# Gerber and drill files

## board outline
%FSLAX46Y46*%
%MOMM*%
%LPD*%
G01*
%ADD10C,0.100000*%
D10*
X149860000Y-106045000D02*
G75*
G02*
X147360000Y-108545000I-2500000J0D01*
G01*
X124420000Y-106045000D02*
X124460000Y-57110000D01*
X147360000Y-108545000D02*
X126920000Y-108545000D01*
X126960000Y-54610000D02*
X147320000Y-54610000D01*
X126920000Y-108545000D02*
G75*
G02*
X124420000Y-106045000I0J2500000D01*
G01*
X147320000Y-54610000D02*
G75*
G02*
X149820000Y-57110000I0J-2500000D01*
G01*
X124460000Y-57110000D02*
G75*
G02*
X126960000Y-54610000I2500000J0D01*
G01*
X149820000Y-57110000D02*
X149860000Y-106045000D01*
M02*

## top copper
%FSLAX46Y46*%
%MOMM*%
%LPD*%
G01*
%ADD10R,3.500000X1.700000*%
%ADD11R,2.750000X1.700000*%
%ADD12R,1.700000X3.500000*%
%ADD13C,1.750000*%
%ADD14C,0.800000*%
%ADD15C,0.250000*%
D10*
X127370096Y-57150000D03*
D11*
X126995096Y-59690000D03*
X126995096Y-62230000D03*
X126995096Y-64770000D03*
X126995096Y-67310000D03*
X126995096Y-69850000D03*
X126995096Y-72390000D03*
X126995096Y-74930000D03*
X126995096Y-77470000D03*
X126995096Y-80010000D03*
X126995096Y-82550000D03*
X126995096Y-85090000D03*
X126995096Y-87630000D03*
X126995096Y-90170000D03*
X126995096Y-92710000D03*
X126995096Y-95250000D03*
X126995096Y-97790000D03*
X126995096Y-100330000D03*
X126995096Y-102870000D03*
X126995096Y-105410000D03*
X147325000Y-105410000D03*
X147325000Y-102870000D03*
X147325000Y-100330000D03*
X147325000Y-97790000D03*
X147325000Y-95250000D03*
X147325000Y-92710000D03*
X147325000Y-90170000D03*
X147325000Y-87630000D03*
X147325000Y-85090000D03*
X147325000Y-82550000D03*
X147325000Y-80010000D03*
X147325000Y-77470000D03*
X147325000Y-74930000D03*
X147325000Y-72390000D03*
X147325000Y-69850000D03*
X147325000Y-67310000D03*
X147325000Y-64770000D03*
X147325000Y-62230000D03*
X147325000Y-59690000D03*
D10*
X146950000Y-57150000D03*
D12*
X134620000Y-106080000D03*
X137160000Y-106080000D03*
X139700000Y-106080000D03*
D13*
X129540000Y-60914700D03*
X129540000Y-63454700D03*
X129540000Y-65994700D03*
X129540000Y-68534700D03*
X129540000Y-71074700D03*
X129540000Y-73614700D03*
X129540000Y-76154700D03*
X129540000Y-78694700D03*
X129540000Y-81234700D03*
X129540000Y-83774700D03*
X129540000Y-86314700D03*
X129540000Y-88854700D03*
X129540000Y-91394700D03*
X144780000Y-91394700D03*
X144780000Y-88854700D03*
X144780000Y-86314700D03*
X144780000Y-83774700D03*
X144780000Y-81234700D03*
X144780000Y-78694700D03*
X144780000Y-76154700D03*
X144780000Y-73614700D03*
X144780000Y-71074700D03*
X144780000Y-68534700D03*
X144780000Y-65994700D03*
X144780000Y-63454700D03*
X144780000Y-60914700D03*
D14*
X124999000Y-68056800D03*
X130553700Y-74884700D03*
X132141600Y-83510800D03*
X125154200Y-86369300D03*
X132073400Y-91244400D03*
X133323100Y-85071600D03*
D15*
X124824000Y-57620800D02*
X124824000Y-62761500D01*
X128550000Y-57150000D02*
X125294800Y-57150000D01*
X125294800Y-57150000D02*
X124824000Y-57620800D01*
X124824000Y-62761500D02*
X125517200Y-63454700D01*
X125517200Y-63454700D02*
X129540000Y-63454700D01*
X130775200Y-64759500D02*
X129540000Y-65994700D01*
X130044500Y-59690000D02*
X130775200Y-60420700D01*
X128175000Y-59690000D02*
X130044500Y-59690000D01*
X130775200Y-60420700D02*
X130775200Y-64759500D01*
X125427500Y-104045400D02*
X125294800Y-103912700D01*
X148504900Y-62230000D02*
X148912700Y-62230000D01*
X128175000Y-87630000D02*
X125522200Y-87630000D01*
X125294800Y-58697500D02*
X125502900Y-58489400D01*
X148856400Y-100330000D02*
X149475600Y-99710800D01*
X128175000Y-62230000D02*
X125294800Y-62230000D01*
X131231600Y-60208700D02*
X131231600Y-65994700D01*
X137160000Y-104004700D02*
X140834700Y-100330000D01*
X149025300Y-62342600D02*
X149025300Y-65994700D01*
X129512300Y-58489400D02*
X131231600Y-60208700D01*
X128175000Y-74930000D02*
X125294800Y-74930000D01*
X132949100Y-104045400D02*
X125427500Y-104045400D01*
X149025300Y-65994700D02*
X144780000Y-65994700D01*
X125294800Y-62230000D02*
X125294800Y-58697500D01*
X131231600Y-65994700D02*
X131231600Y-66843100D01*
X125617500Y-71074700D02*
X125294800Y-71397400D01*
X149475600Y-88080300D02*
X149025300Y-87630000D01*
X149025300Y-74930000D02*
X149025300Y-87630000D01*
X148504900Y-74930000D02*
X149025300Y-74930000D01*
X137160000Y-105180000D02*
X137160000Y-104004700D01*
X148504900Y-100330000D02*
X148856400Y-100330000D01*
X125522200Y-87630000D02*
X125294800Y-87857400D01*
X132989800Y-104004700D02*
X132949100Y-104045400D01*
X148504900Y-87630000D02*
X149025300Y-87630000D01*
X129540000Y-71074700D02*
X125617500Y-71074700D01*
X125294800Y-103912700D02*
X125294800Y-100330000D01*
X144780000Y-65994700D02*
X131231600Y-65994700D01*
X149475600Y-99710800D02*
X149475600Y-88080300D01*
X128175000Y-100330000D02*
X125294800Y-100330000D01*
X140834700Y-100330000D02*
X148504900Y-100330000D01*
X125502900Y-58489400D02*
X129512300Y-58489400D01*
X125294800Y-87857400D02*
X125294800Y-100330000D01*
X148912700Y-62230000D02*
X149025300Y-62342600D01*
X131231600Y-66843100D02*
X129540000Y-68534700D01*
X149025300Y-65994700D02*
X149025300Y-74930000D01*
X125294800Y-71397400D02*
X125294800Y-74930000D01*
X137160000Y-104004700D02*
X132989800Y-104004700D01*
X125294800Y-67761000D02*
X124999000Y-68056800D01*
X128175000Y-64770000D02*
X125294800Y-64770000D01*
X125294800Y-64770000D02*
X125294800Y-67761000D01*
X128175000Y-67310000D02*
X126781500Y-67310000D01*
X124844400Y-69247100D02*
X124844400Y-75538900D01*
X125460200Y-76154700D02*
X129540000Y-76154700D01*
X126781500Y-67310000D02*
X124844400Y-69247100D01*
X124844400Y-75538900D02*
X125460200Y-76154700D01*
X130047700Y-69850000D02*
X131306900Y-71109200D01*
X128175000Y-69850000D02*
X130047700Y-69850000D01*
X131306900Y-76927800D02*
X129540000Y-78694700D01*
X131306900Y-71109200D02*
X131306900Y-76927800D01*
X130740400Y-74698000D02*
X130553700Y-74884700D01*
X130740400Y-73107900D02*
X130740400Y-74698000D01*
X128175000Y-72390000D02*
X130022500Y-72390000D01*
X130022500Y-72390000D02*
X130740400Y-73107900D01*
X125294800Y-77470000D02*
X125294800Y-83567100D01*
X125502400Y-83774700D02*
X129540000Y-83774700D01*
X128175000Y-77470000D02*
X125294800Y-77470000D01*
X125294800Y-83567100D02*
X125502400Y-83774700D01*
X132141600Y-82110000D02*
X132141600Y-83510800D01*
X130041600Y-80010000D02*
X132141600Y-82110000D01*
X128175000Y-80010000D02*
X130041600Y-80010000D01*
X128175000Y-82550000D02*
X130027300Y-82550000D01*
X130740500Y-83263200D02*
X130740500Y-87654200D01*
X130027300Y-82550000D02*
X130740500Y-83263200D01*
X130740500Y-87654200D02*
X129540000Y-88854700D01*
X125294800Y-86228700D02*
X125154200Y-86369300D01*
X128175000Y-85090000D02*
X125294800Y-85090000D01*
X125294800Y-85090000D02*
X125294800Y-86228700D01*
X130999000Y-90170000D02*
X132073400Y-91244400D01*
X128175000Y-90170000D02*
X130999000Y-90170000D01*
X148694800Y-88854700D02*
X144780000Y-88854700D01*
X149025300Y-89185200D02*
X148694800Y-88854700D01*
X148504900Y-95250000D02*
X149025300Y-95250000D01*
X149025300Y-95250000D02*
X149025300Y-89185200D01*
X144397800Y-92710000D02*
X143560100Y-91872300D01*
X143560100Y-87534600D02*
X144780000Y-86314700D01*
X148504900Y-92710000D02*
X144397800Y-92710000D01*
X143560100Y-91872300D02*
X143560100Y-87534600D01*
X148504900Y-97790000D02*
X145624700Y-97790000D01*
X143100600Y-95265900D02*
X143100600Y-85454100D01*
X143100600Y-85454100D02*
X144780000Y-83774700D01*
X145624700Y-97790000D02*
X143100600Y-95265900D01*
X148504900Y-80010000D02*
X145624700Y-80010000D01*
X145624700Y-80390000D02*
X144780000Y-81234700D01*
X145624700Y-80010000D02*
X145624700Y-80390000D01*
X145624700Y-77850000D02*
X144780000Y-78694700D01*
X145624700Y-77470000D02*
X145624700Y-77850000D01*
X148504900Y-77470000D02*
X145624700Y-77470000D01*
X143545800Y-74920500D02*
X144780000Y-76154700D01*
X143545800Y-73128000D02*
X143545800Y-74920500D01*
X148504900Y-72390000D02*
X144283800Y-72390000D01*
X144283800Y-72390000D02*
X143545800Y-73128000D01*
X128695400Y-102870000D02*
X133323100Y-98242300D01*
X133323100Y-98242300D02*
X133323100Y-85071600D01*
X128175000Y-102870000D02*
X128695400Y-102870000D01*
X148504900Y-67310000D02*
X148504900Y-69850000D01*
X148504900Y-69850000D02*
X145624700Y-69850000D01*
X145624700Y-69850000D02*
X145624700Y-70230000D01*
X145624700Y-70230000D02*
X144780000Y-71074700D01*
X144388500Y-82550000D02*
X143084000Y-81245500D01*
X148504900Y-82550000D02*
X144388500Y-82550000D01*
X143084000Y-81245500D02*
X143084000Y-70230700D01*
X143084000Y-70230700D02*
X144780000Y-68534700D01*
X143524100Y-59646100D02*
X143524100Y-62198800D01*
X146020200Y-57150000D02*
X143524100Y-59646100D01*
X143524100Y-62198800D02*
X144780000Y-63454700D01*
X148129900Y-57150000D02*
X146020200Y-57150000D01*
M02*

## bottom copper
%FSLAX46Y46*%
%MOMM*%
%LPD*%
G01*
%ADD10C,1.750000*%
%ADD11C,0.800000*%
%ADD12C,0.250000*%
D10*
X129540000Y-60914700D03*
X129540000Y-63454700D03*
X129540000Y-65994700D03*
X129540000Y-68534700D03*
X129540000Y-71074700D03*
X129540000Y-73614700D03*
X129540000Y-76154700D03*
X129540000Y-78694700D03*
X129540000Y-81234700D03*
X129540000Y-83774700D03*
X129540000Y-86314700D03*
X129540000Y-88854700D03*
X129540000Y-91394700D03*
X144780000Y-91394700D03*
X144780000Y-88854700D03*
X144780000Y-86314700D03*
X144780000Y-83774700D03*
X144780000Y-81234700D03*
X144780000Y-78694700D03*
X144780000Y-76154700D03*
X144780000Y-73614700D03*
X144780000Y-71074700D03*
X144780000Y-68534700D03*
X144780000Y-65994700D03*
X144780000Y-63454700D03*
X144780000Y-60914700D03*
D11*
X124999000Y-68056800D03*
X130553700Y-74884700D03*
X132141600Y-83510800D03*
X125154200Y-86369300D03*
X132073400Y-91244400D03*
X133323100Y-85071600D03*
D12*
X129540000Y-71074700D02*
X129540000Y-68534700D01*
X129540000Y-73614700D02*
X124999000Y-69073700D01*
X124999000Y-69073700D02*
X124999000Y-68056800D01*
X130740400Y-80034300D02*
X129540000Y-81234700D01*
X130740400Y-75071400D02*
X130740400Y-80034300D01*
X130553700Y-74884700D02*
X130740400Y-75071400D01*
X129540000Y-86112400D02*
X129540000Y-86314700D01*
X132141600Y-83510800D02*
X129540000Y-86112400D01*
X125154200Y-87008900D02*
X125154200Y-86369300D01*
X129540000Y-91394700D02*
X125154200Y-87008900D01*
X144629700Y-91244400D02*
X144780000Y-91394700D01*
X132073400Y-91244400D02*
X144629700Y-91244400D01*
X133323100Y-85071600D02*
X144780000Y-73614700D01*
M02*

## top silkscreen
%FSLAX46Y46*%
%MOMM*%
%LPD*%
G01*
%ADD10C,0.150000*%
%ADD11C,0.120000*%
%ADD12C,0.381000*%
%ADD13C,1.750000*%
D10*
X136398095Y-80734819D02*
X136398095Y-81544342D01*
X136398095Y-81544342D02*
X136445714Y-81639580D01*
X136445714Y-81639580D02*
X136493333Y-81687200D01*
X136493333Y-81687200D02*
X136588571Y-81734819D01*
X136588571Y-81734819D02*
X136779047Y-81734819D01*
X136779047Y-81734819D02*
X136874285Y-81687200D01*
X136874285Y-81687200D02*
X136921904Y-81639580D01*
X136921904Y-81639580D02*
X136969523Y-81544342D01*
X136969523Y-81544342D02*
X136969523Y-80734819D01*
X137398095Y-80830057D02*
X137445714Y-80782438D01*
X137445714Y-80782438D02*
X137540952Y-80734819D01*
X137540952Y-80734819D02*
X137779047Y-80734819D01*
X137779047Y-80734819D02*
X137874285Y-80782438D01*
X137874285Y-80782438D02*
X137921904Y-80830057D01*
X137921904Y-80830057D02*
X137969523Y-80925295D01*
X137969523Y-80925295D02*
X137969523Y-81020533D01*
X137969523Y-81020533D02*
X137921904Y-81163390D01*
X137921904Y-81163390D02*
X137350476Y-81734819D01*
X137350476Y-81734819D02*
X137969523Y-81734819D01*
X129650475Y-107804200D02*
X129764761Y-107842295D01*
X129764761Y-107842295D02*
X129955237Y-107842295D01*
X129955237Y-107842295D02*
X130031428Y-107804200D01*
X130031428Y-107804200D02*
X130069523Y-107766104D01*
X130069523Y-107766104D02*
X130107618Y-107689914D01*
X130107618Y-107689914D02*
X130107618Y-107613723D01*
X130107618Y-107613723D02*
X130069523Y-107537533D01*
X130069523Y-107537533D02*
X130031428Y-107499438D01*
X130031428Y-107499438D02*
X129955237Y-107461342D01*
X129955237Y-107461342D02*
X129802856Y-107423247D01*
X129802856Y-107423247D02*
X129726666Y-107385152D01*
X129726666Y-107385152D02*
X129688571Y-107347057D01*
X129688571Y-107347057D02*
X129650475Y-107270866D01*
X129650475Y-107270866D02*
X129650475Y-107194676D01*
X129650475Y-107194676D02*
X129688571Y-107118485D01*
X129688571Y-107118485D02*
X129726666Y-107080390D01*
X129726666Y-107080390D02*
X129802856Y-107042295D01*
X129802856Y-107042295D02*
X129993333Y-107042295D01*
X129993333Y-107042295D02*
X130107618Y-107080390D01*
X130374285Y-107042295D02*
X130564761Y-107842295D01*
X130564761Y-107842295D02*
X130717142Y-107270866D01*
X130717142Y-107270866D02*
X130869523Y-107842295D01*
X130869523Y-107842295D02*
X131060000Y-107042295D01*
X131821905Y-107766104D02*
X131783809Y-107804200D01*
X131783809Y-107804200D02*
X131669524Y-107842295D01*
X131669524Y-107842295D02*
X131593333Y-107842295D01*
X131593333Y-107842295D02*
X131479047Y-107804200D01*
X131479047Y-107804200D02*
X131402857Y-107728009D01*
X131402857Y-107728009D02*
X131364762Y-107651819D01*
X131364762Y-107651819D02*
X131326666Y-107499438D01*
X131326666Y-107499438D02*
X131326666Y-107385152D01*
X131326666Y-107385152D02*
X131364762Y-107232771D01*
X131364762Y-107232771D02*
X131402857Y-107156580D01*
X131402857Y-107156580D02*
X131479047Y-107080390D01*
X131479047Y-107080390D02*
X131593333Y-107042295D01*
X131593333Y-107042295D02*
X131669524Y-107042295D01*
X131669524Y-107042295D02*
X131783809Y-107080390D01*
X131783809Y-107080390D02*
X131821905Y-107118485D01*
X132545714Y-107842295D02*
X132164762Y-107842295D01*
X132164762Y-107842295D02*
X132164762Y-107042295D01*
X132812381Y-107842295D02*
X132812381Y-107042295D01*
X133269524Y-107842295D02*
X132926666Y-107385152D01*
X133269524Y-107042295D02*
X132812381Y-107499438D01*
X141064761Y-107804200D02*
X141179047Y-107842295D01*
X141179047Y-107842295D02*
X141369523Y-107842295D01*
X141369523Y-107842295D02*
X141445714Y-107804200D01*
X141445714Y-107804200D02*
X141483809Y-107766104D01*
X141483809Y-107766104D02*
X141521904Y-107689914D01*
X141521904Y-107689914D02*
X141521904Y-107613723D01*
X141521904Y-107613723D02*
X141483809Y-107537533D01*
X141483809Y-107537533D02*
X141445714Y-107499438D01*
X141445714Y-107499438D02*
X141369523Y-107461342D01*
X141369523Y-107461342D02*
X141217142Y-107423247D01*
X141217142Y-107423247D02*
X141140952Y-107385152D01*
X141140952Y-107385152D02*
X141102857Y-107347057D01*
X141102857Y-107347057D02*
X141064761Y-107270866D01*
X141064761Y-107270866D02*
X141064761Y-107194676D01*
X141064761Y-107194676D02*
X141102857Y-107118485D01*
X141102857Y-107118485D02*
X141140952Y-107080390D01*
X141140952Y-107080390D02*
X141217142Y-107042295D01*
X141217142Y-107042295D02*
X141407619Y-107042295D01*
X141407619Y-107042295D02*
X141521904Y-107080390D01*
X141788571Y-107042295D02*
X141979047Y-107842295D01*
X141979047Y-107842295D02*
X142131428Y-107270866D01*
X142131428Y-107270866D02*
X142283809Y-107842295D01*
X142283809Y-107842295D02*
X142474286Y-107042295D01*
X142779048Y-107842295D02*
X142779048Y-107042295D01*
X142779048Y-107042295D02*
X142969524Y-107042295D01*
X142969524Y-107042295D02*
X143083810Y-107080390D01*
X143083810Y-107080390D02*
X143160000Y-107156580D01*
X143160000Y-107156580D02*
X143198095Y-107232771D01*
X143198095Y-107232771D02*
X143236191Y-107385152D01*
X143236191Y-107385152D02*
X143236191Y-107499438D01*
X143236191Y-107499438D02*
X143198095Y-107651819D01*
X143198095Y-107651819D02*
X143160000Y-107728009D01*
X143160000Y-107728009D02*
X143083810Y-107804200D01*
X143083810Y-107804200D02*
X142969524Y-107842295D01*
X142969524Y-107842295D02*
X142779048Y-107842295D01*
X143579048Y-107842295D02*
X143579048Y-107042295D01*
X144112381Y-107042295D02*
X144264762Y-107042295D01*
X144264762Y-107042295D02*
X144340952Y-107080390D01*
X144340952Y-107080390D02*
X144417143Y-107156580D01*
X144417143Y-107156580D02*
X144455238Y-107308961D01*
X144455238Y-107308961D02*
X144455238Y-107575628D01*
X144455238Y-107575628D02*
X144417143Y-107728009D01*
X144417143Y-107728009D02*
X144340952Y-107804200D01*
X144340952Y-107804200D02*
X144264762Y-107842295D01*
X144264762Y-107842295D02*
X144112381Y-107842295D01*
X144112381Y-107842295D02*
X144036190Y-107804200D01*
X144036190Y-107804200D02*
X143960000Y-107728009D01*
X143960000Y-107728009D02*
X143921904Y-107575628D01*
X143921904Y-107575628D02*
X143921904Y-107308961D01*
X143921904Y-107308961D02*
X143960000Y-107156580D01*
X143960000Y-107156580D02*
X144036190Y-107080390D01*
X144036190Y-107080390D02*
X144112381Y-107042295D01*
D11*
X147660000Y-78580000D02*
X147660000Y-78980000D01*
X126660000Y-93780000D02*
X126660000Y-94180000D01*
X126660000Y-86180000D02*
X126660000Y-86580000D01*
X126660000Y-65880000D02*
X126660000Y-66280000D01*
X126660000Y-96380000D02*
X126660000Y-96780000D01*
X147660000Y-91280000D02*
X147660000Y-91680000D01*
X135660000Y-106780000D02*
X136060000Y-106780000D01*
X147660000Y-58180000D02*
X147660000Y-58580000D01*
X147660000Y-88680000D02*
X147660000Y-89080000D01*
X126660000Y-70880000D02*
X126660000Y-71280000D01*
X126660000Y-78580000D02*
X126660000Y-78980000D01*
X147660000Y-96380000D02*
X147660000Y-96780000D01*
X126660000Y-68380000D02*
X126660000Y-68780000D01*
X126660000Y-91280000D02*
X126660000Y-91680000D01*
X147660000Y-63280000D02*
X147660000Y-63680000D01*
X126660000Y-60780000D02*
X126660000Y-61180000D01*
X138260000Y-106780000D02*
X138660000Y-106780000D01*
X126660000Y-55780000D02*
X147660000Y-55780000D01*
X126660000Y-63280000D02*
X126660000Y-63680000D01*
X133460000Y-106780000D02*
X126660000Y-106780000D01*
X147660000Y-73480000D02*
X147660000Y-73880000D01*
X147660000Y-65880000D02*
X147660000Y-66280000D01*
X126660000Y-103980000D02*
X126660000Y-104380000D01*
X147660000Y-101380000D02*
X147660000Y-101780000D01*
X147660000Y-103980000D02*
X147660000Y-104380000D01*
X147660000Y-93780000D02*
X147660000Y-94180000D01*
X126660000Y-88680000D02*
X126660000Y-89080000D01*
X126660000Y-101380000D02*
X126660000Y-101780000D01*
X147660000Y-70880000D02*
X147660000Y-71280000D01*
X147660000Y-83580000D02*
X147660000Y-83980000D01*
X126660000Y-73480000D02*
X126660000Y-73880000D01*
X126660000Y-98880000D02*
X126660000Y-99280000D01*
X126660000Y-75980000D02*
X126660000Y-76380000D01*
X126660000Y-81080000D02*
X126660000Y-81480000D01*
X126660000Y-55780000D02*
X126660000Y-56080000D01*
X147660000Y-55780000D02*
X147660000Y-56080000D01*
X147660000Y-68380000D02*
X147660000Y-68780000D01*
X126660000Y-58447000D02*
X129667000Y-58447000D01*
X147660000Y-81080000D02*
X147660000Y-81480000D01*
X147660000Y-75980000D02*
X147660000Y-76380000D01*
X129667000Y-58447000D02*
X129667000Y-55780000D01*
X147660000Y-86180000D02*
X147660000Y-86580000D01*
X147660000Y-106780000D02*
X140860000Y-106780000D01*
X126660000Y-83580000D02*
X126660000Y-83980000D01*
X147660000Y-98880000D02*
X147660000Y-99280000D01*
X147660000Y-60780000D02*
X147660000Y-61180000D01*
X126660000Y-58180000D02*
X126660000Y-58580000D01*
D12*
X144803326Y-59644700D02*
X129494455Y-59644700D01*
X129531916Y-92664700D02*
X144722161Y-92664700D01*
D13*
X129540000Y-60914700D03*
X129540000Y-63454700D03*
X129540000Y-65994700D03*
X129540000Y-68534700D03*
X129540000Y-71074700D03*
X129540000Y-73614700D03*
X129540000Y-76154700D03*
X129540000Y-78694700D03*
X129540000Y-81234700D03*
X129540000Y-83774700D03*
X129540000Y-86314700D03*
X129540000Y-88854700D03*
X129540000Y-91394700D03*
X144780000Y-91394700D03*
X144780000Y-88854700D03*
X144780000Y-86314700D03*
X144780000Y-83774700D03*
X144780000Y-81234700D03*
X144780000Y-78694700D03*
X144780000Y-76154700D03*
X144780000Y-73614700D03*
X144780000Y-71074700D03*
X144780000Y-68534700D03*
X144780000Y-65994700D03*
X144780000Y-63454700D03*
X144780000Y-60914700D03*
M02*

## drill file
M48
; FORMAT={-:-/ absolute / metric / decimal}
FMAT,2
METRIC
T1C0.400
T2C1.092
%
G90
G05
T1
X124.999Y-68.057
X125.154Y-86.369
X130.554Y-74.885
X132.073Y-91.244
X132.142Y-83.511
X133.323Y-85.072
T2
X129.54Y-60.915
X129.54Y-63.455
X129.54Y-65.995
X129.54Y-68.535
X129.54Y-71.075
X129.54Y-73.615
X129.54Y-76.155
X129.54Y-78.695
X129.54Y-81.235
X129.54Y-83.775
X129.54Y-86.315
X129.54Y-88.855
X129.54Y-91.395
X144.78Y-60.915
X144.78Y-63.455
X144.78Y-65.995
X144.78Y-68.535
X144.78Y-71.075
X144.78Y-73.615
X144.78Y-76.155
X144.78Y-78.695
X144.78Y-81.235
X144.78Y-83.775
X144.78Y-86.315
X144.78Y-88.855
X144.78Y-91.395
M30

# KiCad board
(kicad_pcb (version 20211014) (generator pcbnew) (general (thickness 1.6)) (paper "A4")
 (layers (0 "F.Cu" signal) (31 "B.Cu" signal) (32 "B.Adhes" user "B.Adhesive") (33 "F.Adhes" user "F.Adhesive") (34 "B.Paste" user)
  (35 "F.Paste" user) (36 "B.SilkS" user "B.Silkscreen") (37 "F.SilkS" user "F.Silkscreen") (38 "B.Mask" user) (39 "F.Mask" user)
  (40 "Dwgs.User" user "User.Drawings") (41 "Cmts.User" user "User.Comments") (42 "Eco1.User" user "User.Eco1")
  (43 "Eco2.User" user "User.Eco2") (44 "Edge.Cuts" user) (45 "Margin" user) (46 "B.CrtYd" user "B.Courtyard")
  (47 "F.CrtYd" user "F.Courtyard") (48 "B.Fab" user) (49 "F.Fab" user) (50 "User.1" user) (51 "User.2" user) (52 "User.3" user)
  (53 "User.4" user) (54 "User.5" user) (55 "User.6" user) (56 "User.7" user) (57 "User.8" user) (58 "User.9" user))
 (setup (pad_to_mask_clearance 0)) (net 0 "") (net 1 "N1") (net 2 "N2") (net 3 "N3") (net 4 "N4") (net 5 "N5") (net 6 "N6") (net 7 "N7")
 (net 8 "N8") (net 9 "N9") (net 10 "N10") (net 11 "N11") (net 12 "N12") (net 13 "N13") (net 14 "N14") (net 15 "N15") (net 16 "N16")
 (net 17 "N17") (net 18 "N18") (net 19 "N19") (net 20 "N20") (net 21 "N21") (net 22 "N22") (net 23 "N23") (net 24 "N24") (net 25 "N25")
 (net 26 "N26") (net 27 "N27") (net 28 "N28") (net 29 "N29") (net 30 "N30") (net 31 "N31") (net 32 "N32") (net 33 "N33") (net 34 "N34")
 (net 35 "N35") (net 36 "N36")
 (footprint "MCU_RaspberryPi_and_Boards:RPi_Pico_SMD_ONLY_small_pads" (layer "F.Cu") (at 137.16 81.28)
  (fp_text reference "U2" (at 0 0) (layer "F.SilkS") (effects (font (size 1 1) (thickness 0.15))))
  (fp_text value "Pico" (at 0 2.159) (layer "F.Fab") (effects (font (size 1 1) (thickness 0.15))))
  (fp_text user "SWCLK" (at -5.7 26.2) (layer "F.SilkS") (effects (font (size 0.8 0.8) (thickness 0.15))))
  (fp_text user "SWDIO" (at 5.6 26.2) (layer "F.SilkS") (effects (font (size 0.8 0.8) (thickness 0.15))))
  (fp_line (start 10.5 -2.7) (end 10.5 -2.3) (layer "F.SilkS") (width 0.12))
  (fp_line (start -10.5 12.5) (end -10.5 12.9) (layer "F.SilkS") (width 0.12))
  (fp_line (start -10.5 4.9) (end -10.5 5.3) (layer "F.SilkS") (width 0.12))
  (fp_line (start -10.5 -15.4) (end -10.5 -15) (layer "F.SilkS") (width 0.12))
  (fp_line (start -10.5 15.1) (end -10.5 15.5) (layer "F.SilkS") (width 0.12))
  (fp_line (start 10.5 10) (end 10.5 10.4) (layer "F.SilkS") (width 0.12))
  (fp_line (start -1.5 25.5) (end -1.1 25.5) (layer "F.SilkS") (width 0.12))
  (fp_line (start 10.5 -23.1) (end 10.5 -22.7) (layer "F.SilkS") (width 0.12))
  (fp_line (start 10.5 7.4) (end 10.5 7.8) (layer "F.SilkS") (width 0.12))
  (fp_line (start -10.5 -10.4) (end -10.5 -10) (layer "F.SilkS") (width 0.12))
  (fp_line (start -10.5 -2.7) (end -10.5 -2.3) (layer "F.SilkS") (width 0.12))
  (fp_line (start 10.5 15.1) (end 10.5 15.5) (layer "F.SilkS") (width 0.12))
  (fp_line (start -10.5 -12.9) (end -10.5 -12.5) (layer "F.SilkS") (width 0.12))
  (fp_line (start -10.5 10) (end -10.5 10.4) (layer "F.SilkS") (width 0.12))
  (fp_line (start 10.5 -18) (end 10.5 -17.6) (layer "F.SilkS") (width 0.12))
  (fp_line (start -10.5 -20.5) (end -10.5 -20.1) (layer "F.SilkS") (width 0.12))
  (fp_line (start 1.1 25.5) (end 1.5 25.5) (layer "F.SilkS") (width 0.12))
  (fp_line (start -10.5 -25.5) (end 10.5 -25.5) (layer "F.SilkS") (width 0.12))
  (fp_line (start -10.5 -18) (end -10.5 -17.6) (layer "F.SilkS") (width 0.12))
  (fp_line (start -3.7 25.5) (end -10.5 25.5) (layer "F.SilkS") (width 0.12))
  (fp_line (start 10.5 -7.8) (end 10.5 -7.4) (layer "F.SilkS") (width 0.12))
  (fp_line (start 10.5 -15.4) (end 10.5 -15) (layer "F.SilkS") (width 0.12))
  (fp_line (start -10.5 22.7) (end -10.5 23.1) (layer "F.SilkS") (width 0.12))
  (fp_line (start 10.5 20.1) (end 10.5 20.5) (layer "F.SilkS") (width 0.12))
  (fp_line (start 10.5 22.7) (end 10.5 23.1) (layer "F.SilkS") (width 0.12))
  (fp_line (start 10.5 12.5) (end 10.5 12.9) (layer "F.SilkS") (width 0.12))
  (fp_line (start -10.5 7.4) (end -10.5 7.8) (layer "F.SilkS") (width 0.12))
  (fp_line (start -10.5 20.1) (end -10.5 20.5) (layer "F.SilkS") (width 0.12))
  (fp_line (start 10.5 -10.4) (end 10.5 -10) (layer "F.SilkS") (width 0.12))
  (fp_line (start 10.5 2.3) (end 10.5 2.7) (layer "F.SilkS") (width 0.12))
  (fp_line (start -10.5 -7.8) (end -10.5 -7.4) (layer "F.SilkS") (width 0.12))
  (fp_line (start -10.5 17.6) (end -10.5 18) (layer "F.SilkS") (width 0.12))
  (fp_line (start -10.5 -5.3) (end -10.5 -4.9) (layer "F.SilkS") (width 0.12))
  (fp_line (start -10.5 -0.2) (end -10.5 0.2) (layer "F.SilkS") (width 0.12))
  (fp_line (start -10.5 -25.5) (end -10.5 -25.2) (layer "F.SilkS") (width 0.12))
  (fp_line (start 10.5 -25.5) (end 10.5 -25.2) (layer "F.SilkS") (width 0.12))
  (fp_line (start 10.5 -12.9) (end 10.5 -12.5) (layer "F.SilkS") (width 0.12))
  (fp_line (start -10.5 -22.833) (end -7.493 -22.833) (layer "F.SilkS") (width 0.12))
  (fp_line (start 10.5 -0.2) (end 10.5 0.2) (layer "F.SilkS") (width 0.12))
  (fp_line (start 10.5 -5.3) (end 10.5 -4.9) (layer "F.SilkS") (width 0.12))
  (fp_line (start -7.493 -22.833) (end -7.493 -25.5) (layer "F.SilkS") (width 0.12))
  (fp_line (start 10.5 4.9) (end 10.5 5.3) (layer "F.SilkS") (width 0.12))
  (fp_line (start 10.5 25.5) (end 3.7 25.5) (layer "F.SilkS") (width 0.12))
  (fp_line (start -10.5 2.3) (end -10.5 2.7) (layer "F.SilkS") (width 0.12))
  (fp_line (start 10.5 17.6) (end 10.5 18) (layer "F.SilkS") (width 0.12))
  (fp_line (start 10.5 -20.5) (end 10.5 -20.1) (layer "F.SilkS") (width 0.12))
  (fp_line (start -10.5 -23.1) (end -10.5 -22.7) (layer "F.SilkS") (width 0.12))
  (pad "1" smd rect (at -8.609992 -24.13) (size 3.5 1.7) (drill (offset -1.179912 0)) (layers "F.Cu" "F.Mask") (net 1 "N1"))
  (pad "2" smd rect (at -8.984992 -21.59) (size 2.75 1.7) (drill (offset -1.179912 0)) (layers "F.Cu" "F.Mask") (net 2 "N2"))
  (pad "3" smd rect (at -8.984992 -19.05) (size 2.75 1.7) (drill (offset -1.179912 0)) (layers "F.Cu" "F.Mask") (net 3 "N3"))
  (pad "4" smd rect (at -8.984992 -16.51) (size 2.75 1.7) (drill (offset -1.179912 0)) (layers "F.Cu" "F.Mask") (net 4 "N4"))
  (pad "5" smd rect (at -8.984992 -13.97) (size 2.75 1.7) (drill (offset -1.179912 0)) (layers "F.Cu" "F.Mask") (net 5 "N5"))
  (pad "6" smd rect (at -8.984992 -11.43) (size 2.75 1.7) (drill (offset -1.179912 0)) (layers "F.Cu" "F.Mask") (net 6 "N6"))
  (pad "7" smd rect (at -8.984992 -8.89) (size 2.75 1.7) (drill (offset -1.179912 0)) (layers "F.Cu" "F.Mask") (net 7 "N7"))
  (pad "8" smd rect (at -8.984992 -6.35) (size 2.75 1.7) (drill (offset -1.179912 0)) (layers "F.Cu" "F.Mask") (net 3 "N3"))
  (pad "9" smd rect (at -8.984992 -3.81) (size 2.75 1.7) (drill (offset -1.179912 0)) (layers "F.Cu" "F.Mask") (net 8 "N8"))
  (pad "10" smd rect (at -8.984992 -1.27) (size 2.75 1.7) (drill (offset -1.179912 0)) (layers "F.Cu" "F.Mask") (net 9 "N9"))
  (pad "11" smd rect (at -8.984992 1.27) (size 2.75 1.7) (drill (offset -1.179912 0)) (layers "F.Cu" "F.Mask") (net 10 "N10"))
  (pad "12" smd rect (at -8.984992 3.81) (size 2.75 1.7) (drill (offset -1.179912 0)) (layers "F.Cu" "F.Mask") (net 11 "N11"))
  (pad "13" smd rect (at -8.984992 6.35) (size 2.75 1.7) (drill (offset -1.179912 0)) (layers "F.Cu" "F.Mask") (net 3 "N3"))
  (pad "14" smd rect (at -8.984992 8.89) (size 2.75 1.7) (drill (offset -1.179912 0)) (layers "F.Cu" "F.Mask") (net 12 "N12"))
  (pad "15" smd rect (at -8.984992 11.43) (size 2.75 1.7) (drill (offset -1.179912 0)) (layers "F.Cu" "F.Mask") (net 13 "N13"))
  (pad "16" smd rect (at -8.984992 13.97) (size 2.75 1.7) (drill (offset -1.179912 0)) (layers "F.Cu" "F.Mask") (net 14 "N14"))
  (pad "17" smd rect (at -8.984992 16.51) (size 2.75 1.7) (drill (offset -1.179912 0)) (layers "F.Cu" "F.Mask") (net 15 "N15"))
  (pad "18" smd rect (at -8.984992 19.05) (size 2.75 1.7) (drill (offset -1.179912 0)) (layers "F.Cu" "F.Mask") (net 3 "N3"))
  (pad "19" smd rect (at -8.984992 21.59) (size 2.75 1.7) (drill (offset -1.179912 0)) (layers "F.Cu" "F.Mask") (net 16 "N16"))
  (pad "20" smd rect (at -8.984992 24.13) (size 2.75 1.7) (drill (offset -1.179912 0)) (layers "F.Cu" "F.Mask") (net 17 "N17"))
  (pad "21" smd rect (at 11.344912 24.13) (size 2.75 1.7) (drill (offset -1.179912 0)) (layers "F.Cu" "F.Mask") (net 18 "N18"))
  (pad "22" smd rect (at 11.344912 21.59) (size 2.75 1.7) (drill (offset -1.179912 0)) (layers "F.Cu" "F.Mask") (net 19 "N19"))
  (pad "23" smd rect (at 11.344912 19.05) (size 2.75 1.7) (drill (offset -1.179912 0)) (layers "F.Cu" "F.Mask") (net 3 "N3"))
  (pad "24" smd rect (at 11.344912 16.51) (size 2.75 1.7) (drill (offset -1.179912 0)) (layers "F.Cu" "F.Mask") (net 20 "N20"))
  (pad "25" smd rect (at 11.344912 13.97) (size 2.75 1.7) (drill (offset -1.179912 0)) (layers "F.Cu" "F.Mask") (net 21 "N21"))
  (pad "26" smd rect (at 11.344912 11.43) (size 2.75 1.7) (drill (offset -1.179912 0)) (layers "F.Cu" "F.Mask") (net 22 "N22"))
  (pad "27" smd rect (at 11.344912 8.89) (size 2.75 1.7) (drill (offset -1.179912 0)) (layers "F.Cu" "F.Mask") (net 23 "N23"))
  (pad "28" smd rect (at 11.344912 6.35) (size 2.75 1.7) (drill (offset -1.179912 0)) (layers "F.Cu" "F.Mask") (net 3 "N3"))
  (pad "29" smd rect (at 11.344912 3.81) (size 2.75 1.7) (drill (offset -1.179912 0)) (layers "F.Cu" "F.Mask") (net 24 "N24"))
  (pad "30" smd rect (at 11.344912 1.27) (size 2.75 1.7) (drill (offset -1.179912 0)) (layers "F.Cu" "F.Mask") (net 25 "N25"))
  (pad "31" smd rect (at 11.344912 -1.27) (size 2.75 1.7) (drill (offset -1.179912 0)) (layers "F.Cu" "F.Mask") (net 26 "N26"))
  (pad "32" smd rect (at 11.344912 -3.81) (size 2.75 1.7) (drill (offset -1.179912 0)) (layers "F.Cu" "F.Mask") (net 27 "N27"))
  (pad "33" smd rect (at 11.344912 -6.35) (size 2.75 1.7) (drill (offset -1.179912 0)) (layers "F.Cu" "F.Mask") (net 3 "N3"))
  (pad "34" smd rect (at 11.344912 -8.89) (size 2.75 1.7) (drill (offset -1.179912 0)) (layers "F.Cu" "F.Mask") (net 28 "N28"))
  (pad "35" smd rect (at 11.344912 -11.43) (size 2.75 1.7) (drill (offset -1.179912 0)) (layers "F.Cu" "F.Mask") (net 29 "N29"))
  (pad "36" smd rect (at 11.344912 -13.97) (size 2.75 1.7) (drill (offset -1.179912 0)) (layers "F.Cu" "F.Mask") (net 29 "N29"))
  (pad "37" smd rect (at 11.344912 -16.51) (size 2.75 1.7) (drill (offset -1.179912 0)) (layers "F.Cu" "F.Mask") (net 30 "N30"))
  (pad "38" smd rect (at 11.344912 -19.05) (size 2.75 1.7) (drill (offset -1.179912 0)) (layers "F.Cu" "F.Mask") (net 3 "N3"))
  (pad "39" smd rect (at 11.344912 -21.59) (size 2.75 1.7) (drill (offset -1.179912 0)) (layers "F.Cu" "F.Mask") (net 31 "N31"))
  (pad "40" smd rect (at 10.969912 -24.13) (size 3.5 1.7) (drill (offset -1.179912 0)) (layers "F.Cu" "F.Mask") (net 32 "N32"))
  (pad "41" smd rect (at -2.54 23.9 90) (size 3.5 1.7) (drill (offset -0.9 0)) (layers "F.Cu" "F.Mask") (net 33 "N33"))
  (pad "42" smd rect (at 0 23.9 90) (size 3.5 1.7) (drill (offset -0.9 0)) (layers "F.Cu" "F.Mask") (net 3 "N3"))
  (pad "43" smd rect (at 2.54 23.9 90) (size 3.5 1.7) (drill (offset -0.9 0)) (layers "F.Cu" "F.Mask") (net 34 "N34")))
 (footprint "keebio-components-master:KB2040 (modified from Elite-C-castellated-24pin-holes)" (layer "B.Cu") (at 137.16 77.4247 -90)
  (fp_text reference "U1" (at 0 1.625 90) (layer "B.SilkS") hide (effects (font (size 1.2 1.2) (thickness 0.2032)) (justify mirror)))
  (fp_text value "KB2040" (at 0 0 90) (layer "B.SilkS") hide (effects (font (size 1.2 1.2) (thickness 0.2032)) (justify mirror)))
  (fp_line (start -17.78 -7.643326) (end -17.78 7.665545) (layer "F.SilkS") (width 0.381))
  (fp_line (start 15.24 7.628084) (end 15.24 -7.562161) (layer "F.SilkS") (width 0.381))
  (pad "0" thru_hole circle (at -16.51 7.62 90) (size 1.75 1.75) (drill 1.0922) (layers *.Cu *.SilkS *.Mask) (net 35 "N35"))
  (pad "1" thru_hole circle (at -13.97 7.62 90) (size 1.75 1.75) (drill 1.0922) (layers *.Cu *.SilkS *.Mask) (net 1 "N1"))
  (pad "2" thru_hole circle (at -11.43 7.62 90) (size 1.75 1.75) (drill 1.0922) (layers *.Cu *.SilkS *.Mask) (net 2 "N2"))
  (pad "3" thru_hole circle (at -8.89 7.62 90) (size 1.75 1.75) (drill 1.0922) (layers *.Cu *.SilkS *.Mask) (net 3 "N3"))
  (pad "4" thru_hole circle (at -6.35 7.62 90) (size 1.75 1.75) (drill 1.0922) (layers *.Cu *.SilkS *.Mask) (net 3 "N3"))
  (pad "5" thru_hole circle (at -3.81 7.62 90) (size 1.75 1.75) (drill 1.0922) (layers *.Cu *.SilkS *.Mask) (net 4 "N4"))
  (pad "6" thru_hole circle (at -1.27 7.62 90) (size 1.75 1.75) (drill 1.0922) (layers *.Cu *.SilkS *.Mask) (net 5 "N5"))
  (pad "7" thru_hole circle (at 1.27 7.62 90) (size 1.75 1.75) (drill 1.0922) (layers *.Cu *.SilkS *.Mask) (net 6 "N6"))
  (pad "8" thru_hole circle (at 3.81 7.62 90) (size 1.75 1.75) (drill 1.0922) (layers *.Cu *.SilkS *.Mask) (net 7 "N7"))
  (pad "9" thru_hole circle (at 6.35 7.62 90) (size 1.75 1.75) (drill 1.0922) (layers *.Cu *.SilkS *.Mask) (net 8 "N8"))
  (pad "10" thru_hole circle (at 8.89 7.62 90) (size 1.75 1.75) (drill 1.0922) (layers *.Cu *.SilkS *.Mask) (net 9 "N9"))
  (pad "11" thru_hole circle (at 11.43 7.62 90) (size 1.75 1.75) (drill 1.0922) (layers *.Cu *.SilkS *.Mask) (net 10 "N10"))
  (pad "12" thru_hole circle (at 13.97 7.62 90) (size 1.75 1.75) (drill 1.0922) (layers *.Cu *.SilkS *.Mask) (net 11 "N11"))
  (pad "13" thru_hole circle (at 13.97 -7.62 90) (size 1.75 1.75) (drill 1.0922) (layers *.Cu *.SilkS *.Mask) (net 12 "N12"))
  (pad "14" thru_hole circle (at 11.43 -7.62 90) (size 1.75 1.75) (drill 1.0922) (layers *.Cu *.SilkS *.Mask) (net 21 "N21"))
  (pad "15" thru_hole circle (at 8.89 -7.62 90) (size 1.75 1.75) (drill 1.0922) (layers *.Cu *.SilkS *.Mask) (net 22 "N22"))
  (pad "16" thru_hole circle (at 6.35 -7.62 90) (size 1.75 1.75) (drill 1.0922) (layers *.Cu *.SilkS *.Mask) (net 20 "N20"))
  (pad "17" thru_hole circle (at 3.81 -7.62 90) (size 1.75 1.75) (drill 1.0922) (layers *.Cu *.SilkS *.Mask) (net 26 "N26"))
  (pad "18" thru_hole circle (at 1.27 -7.62 90) (size 1.75 1.75) (drill 1.0922) (layers *.Cu *.SilkS *.Mask) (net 27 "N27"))
  (pad "19" thru_hole circle (at -1.27 -7.62 90) (size 1.75 1.75) (drill 1.0922) (layers *.Cu *.SilkS *.Mask) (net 28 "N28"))
  (pad "20" thru_hole circle (at -3.81 -7.62 90) (size 1.75 1.75) (drill 1.0922) (layers *.Cu *.SilkS *.Mask) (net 16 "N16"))
  (pad "21" thru_hole circle (at -6.35 -7.62 90) (size 1.75 1.75) (drill 1.0922) (layers *.Cu *.SilkS *.Mask) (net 29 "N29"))
  (pad "22" thru_hole circle (at -8.89 -7.62 90) (size 1.75 1.75) (drill 1.0922) (layers *.Cu *.SilkS *.Mask) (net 25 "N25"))
  (pad "23" thru_hole circle (at -11.43 -7.62 90) (size 1.75 1.75) (drill 1.0922) (layers *.Cu *.SilkS *.Mask) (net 3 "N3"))
  (pad "24" thru_hole circle (at -13.97 -7.62 90) (size 1.75 1.75) (drill 1.0922) (layers *.Cu *.SilkS *.Mask) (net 32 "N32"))
  (pad "25" thru_hole circle (at -16.51 -7.62 90) (size 1.75 1.75) (drill 1.0922) (layers *.Cu *.SilkS *.Mask) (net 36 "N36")))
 (gr_arc (start 149.86 106.045) (mid 149.127767 107.812767) (end 147.36 108.545) (layer "Edge.Cuts") (width 0.1))
 (gr_line (start 124.42 106.045) (end 124.46 57.11) (layer "Edge.Cuts") (width 0.1))
 (gr_line (start 147.36 108.545) (end 126.92 108.545) (layer "Edge.Cuts") (width 0.1))
 (gr_line (start 126.96 54.61) (end 147.32 54.61) (layer "Edge.Cuts") (width 0.1))
 (gr_arc (start 126.92 108.545) (mid 125.152233 107.812767) (end 124.42 106.045) (layer "Edge.Cuts") (width 0.1))
 (gr_arc (start 147.32 54.61) (mid 149.087767 55.342233) (end 149.82 57.11) (layer "Edge.Cuts") (width 0.1))
 (gr_arc (start 124.46 57.11) (mid 125.192233 55.342233) (end 126.96 54.61) (layer "Edge.Cuts") (width 0.1))
 (gr_line (start 149.82 57.11) (end 149.86 106.045) (layer "Edge.Cuts") (width 0.1))
 (segment (start 124.824 57.6208) (end 124.824 62.7615) (width 0.25) (layer "F.Cu") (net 1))
 (segment (start 128.55 57.15) (end 125.2948 57.15) (width 0.25) (layer "F.Cu") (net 1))
 (segment (start 125.2948 57.15) (end 124.824 57.6208) (width 0.25) (layer "F.Cu") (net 1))
 (segment (start 124.824 62.7615) (end 125.5172 63.4547) (width 0.25) (layer "F.Cu") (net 1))
 (segment (start 125.5172 63.4547) (end 129.54 63.4547) (width 0.25) (layer "F.Cu") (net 1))
 (segment (start 130.7752 64.7595) (end 129.54 65.9947) (width 0.25) (layer "F.Cu") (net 2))
 (segment (start 130.0445 59.69) (end 130.7752 60.4207) (width 0.25) (layer "F.Cu") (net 2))
 (segment (start 128.175 59.69) (end 130.0445 59.69) (width 0.25) (layer "F.Cu") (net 2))
 (segment (start 130.7752 60.4207) (end 130.7752 64.7595) (width 0.25) (layer "F.Cu") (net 2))
 (segment (start 125.4275 104.0454) (end 125.2948 103.9127) (width 0.25) (layer "F.Cu") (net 3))
 (segment (start 148.5049 62.23) (end 148.9127 62.23) (width 0.25) (layer "F.Cu") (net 3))
 (segment (start 128.175 87.63) (end 125.5222 87.63) (width 0.25) (layer "F.Cu") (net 3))
 (segment (start 125.2948 58.6975) (end 125.5029 58.4894) (width 0.25) (layer "F.Cu") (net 3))
 (segment (start 148.8564 100.33) (end 149.4756 99.7108) (width 0.25) (layer "F.Cu") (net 3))
 (segment (start 128.175 62.23) (end 125.2948 62.23) (width 0.25) (layer "F.Cu") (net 3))
 (segment (start 131.2316 60.2087) (end 131.2316 65.9947) (width 0.25) (layer "F.Cu") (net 3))
 (segment (start 137.16 104.0047) (end 140.8347 100.33) (width 0.25) (layer "F.Cu") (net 3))
 (segment (start 149.0253 62.3426) (end 149.0253 65.9947) (width 0.25) (layer "F.Cu") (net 3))
 (segment (start 129.5123 58.4894) (end 131.2316 60.2087) (width 0.25) (layer "F.Cu") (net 3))
 (segment (start 128.175 74.93) (end 125.2948 74.93) (width 0.25) (layer "F.Cu") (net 3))
 (segment (start 132.9491 104.0454) (end 125.4275 104.0454) (width 0.25) (layer "F.Cu") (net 3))
 (segment (start 149.0253 65.9947) (end 144.78 65.9947) (width 0.25) (layer "F.Cu") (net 3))
 (segment (start 125.2948 62.23) (end 125.2948 58.6975) (width 0.25) (layer "F.Cu") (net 3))
 (segment (start 131.2316 65.9947) (end 131.2316 66.8431) (width 0.25) (layer "F.Cu") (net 3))
 (segment (start 125.6175 71.0747) (end 125.2948 71.3974) (width 0.25) (layer "F.Cu") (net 3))
 (segment (start 149.4756 88.0803) (end 149.0253 87.63) (width 0.25) (layer "F.Cu") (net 3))
 (segment (start 149.0253 74.93) (end 149.0253 87.63) (width 0.25) (layer "F.Cu") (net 3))
 (segment (start 148.5049 74.93) (end 149.0253 74.93) (width 0.25) (layer "F.Cu") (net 3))
 (segment (start 137.16 105.18) (end 137.16 104.0047) (width 0.25) (layer "F.Cu") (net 3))
 (segment (start 148.5049 100.33) (end 148.8564 100.33) (width 0.25) (layer "F.Cu") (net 3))
 (segment (start 125.5222 87.63) (end 125.2948 87.8574) (width 0.25) (layer "F.Cu") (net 3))
 (segment (start 132.9898 104.0047) (end 132.9491 104.0454) (width 0.25) (layer "F.Cu") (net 3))
 (segment (start 148.5049 87.63) (end 149.0253 87.63) (width 0.25) (layer "F.Cu") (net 3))
 (segment (start 129.54 71.0747) (end 125.6175 71.0747) (width 0.25) (layer "F.Cu") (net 3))
 (segment (start 125.2948 103.9127) (end 125.2948 100.33) (width 0.25) (layer "F.Cu") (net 3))
 (segment (start 144.78 65.9947) (end 131.2316 65.9947) (width 0.25) (layer "F.Cu") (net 3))
 (segment (start 149.4756 99.7108) (end 149.4756 88.0803) (width 0.25) (layer "F.Cu") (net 3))
 (segment (start 128.175 100.33) (end 125.2948 100.33) (width 0.25) (layer "F.Cu") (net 3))
 (segment (start 140.8347 100.33) (end 148.5049 100.33) (width 0.25) (layer "F.Cu") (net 3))
 (segment (start 125.5029 58.4894) (end 129.5123 58.4894) (width 0.25) (layer "F.Cu") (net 3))
 (segment (start 125.2948 87.8574) (end 125.2948 100.33) (width 0.25) (layer "F.Cu") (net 3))
 (segment (start 148.9127 62.23) (end 149.0253 62.3426) (width 0.25) (layer "F.Cu") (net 3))
 (segment (start 131.2316 66.8431) (end 129.54 68.5347) (width 0.25) (layer "F.Cu") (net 3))
 (segment (start 149.0253 65.9947) (end 149.0253 74.93) (width 0.25) (layer "F.Cu") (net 3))
 (segment (start 125.2948 71.3974) (end 125.2948 74.93) (width 0.25) (layer "F.Cu") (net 3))
 (segment (start 137.16 104.0047) (end 132.9898 104.0047) (width 0.25) (layer "F.Cu") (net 3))
 (segment (start 129.54 71.0747) (end 129.54 68.5347) (width 0.25) (layer "B.Cu") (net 3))
 (segment (start 125.2948 67.761) (end 124.999 68.0568) (width 0.25) (layer "F.Cu") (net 4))
 (segment (start 128.175 64.77) (end 125.2948 64.77) (width 0.25) (layer "F.Cu") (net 4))
 (segment (start 125.2948 64.77) (end 125.2948 67.761) (width 0.25) (layer "F.Cu") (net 4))
 (via (at 124.999 68.0568) (size 0.8) (drill 0.4) (layers "F.Cu" "B.Cu") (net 4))
 (segment (start 129.54 73.6147) (end 124.999 69.0737) (width 0.25) (layer "B.Cu") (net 4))
 (segment (start 124.999 69.0737) (end 124.999 68.0568) (width 0.25) (layer "B.Cu") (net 4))
 (segment (start 128.175 67.31) (end 126.7815 67.31) (width 0.25) (layer "F.Cu") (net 5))
 (segment (start 124.8444 69.2471) (end 124.8444 75.5389) (width 0.25) (layer "F.Cu") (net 5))
 (segment (start 125.4602 76.1547) (end 129.54 76.1547) (width 0.25) (layer "F.Cu") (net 5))
 (segment (start 126.7815 67.31) (end 124.8444 69.2471) (width 0.25) (layer "F.Cu") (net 5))
 (segment (start 124.8444 75.5389) (end 125.4602 76.1547) (width 0.25) (layer "F.Cu") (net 5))
 (segment (start 130.0477 69.85) (end 131.3069 71.1092) (width 0.25) (layer "F.Cu") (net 6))
 (segment (start 128.175 69.85) (end 130.0477 69.85) (width 0.25) (layer "F.Cu") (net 6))
 (segment (start 131.3069 76.9278) (end 129.54 78.6947) (width 0.25) (layer "F.Cu") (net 6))
 (segment (start 131.3069 71.1092) (end 131.3069 76.9278) (width 0.25) (layer "F.Cu") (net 6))
 (segment (start 130.7404 74.698) (end 130.5537 74.8847) (width 0.25) (layer "F.Cu") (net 7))
 (segment (start 130.7404 73.1079) (end 130.7404 74.698) (width 0.25) (layer "F.Cu") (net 7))
 (segment (start 128.175 72.39) (end 130.0225 72.39) (width 0.25) (layer "F.Cu") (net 7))
 (segment (start 130.0225 72.39) (end 130.7404 73.1079) (width 0.25) (layer "F.Cu") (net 7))
 (via (at 130.5537 74.8847) (size 0.8) (drill 0.4) (layers "F.Cu" "B.Cu") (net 7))
 (segment (start 130.7404 80.0343) (end 129.54 81.2347) (width 0.25) (layer "B.Cu") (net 7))
 (segment (start 130.7404 75.0714) (end 130.7404 80.0343) (width 0.25) (layer "B.Cu") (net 7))
 (segment (start 130.5537 74.8847) (end 130.7404 75.0714) (width 0.25) (layer "B.Cu") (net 7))
 (segment (start 125.2948 77.47) (end 125.2948 83.5671) (width 0.25) (layer "F.Cu") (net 8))
 (segment (start 125.5024 83.7747) (end 129.54 83.7747) (width 0.25) (layer "F.Cu") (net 8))
 (segment (start 128.175 77.47) (end 125.2948 77.47) (width 0.25) (layer "F.Cu") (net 8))
 (segment (start 125.2948 83.5671) (end 125.5024 83.7747) (width 0.25) (layer "F.Cu") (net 8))
 (segment (start 132.1416 82.11) (end 132.1416 83.5108) (width 0.25) (layer "F.Cu") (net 9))
 (segment (start 130.0416 80.01) (end 132.1416 82.11) (width 0.25) (layer "F.Cu") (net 9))
 (segment (start 128.175 80.01) (end 130.0416 80.01) (width 0.25) (layer "F.Cu") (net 9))
 (via (at 132.1416 83.5108) (size 0.8) (drill 0.4) (layers "F.Cu" "B.Cu") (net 9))
 (segment (start 129.54 86.1124) (end 129.54 86.3147) (width 0.25) (layer "B.Cu") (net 9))
 (segment (start 132.1416 83.5108) (end 129.54 86.1124) (width 0.25) (layer "B.Cu") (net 9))
 (segment (start 128.175 82.55) (end 130.0273 82.55) (width 0.25) (layer "F.Cu") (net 10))
 (segment (start 130.7405 83.2632) (end 130.7405 87.6542) (width 0.25) (layer "F.Cu") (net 10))
 (segment (start 130.0273 82.55) (end 130.7405 83.2632) (width 0.25) (layer "F.Cu") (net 10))
 (segment (start 130.7405 87.6542) (end 129.54 88.8547) (width 0.25) (layer "F.Cu") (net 10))
 (segment (start 125.2948 86.2287) (end 125.1542 86.3693) (width 0.25) (layer "F.Cu") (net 11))
 (segment (start 128.175 85.09) (end 125.2948 85.09) (width 0.25) (layer "F.Cu") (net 11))
 (segment (start 125.2948 85.09) (end 125.2948 86.2287) (width 0.25) (layer "F.Cu") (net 11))
 (via (at 125.1542 86.3693) (size 0.8) (drill 0.4) (layers "F.Cu" "B.Cu") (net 11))
 (segment (start 125.1542 87.0089) (end 125.1542 86.3693) (width 0.25) (layer "B.Cu") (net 11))
 (segment (start 129.54 91.3947) (end 125.1542 87.0089) (width 0.25) (layer "B.Cu") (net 11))
 (segment (start 130.999 90.17) (end 132.0734 91.2444) (width 0.25) (layer "F.Cu") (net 12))
 (segment (start 128.175 90.17) (end 130.999 90.17) (width 0.25) (layer "F.Cu") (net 12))
 (via (at 132.0734 91.2444) (size 0.8) (drill 0.4) (layers "F.Cu" "B.Cu") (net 12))
 (segment (start 144.6297 91.2444) (end 144.78 91.3947) (width 0.25) (layer "B.Cu") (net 12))
 (segment (start 132.0734 91.2444) (end 144.6297 91.2444) (width 0.25) (layer "B.Cu") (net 12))
 (segment (start 148.6948 88.8547) (end 144.78 88.8547) (width 0.25) (layer "F.Cu") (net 21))
 (segment (start 149.0253 89.1852) (end 148.6948 88.8547) (width 0.25) (layer "F.Cu") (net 21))
 (segment (start 148.5049 95.25) (end 149.0253 95.25) (width 0.25) (layer "F.Cu") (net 21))
 (segment (start 149.0253 95.25) (end 149.0253 89.1852) (width 0.25) (layer "F.Cu") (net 21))
 (segment (start 144.3978 92.71) (end 143.5601 91.8723) (width 0.25) (layer "F.Cu") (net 22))
 (segment (start 143.5601 87.5346) (end 144.78 86.3147) (width 0.25) (layer "F.Cu") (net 22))
 (segment (start 148.5049 92.71) (end 144.3978 92.71) (width 0.25) (layer "F.Cu") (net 22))
 (segment (start 143.5601 91.8723) (end 143.5601 87.5346) (width 0.25) (layer "F.Cu") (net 22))
 (segment (start 148.5049 97.79) (end 145.6247 97.79) (width 0.25) (layer "F.Cu") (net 20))
 (segment (start 143.1006 95.2659) (end 143.1006 85.4541) (width 0.25) (layer "F.Cu") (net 20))
 (segment (start 143.1006 85.4541) (end 144.78 83.7747) (width 0.25) (layer "F.Cu") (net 20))
 (segment (start 145.6247 97.79) (end 143.1006 95.2659) (width 0.25) (layer "F.Cu") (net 20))
 (segment (start 148.5049 80.01) (end 145.6247 80.01) (width 0.25) (layer "F.Cu") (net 26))
 (segment (start 145.6247 80.39) (end 144.78 81.2347) (width 0.25) (layer "F.Cu") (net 26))
 (segment (start 145.6247 80.01) (end 145.6247 80.39) (width 0.25) (layer "F.Cu") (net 26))
 (segment (start 145.6247 77.85) (end 144.78 78.6947) (width 0.25) (layer "F.Cu") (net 27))
 (segment (start 145.6247 77.47) (end 145.6247 77.85) (width 0.25) (layer "F.Cu") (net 27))
 (segment (start 148.5049 77.47) (end 145.6247 77.47) (width 0.25) (layer "F.Cu") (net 27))
 (segment (start 143.5458 74.9205) (end 144.78 76.1547) (width 0.25) (layer "F.Cu") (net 28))
 (segment (start 143.5458 73.128) (end 143.5458 74.9205) (width 0.25) (layer "F.Cu") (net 28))
 (segment (start 148.5049 72.39) (end 144.2838 72.39) (width 0.25) (layer "F.Cu") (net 28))
 (segment (start 144.2838 72.39) (end 143.5458 73.128) (width 0.25) (layer "F.Cu") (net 28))
 (segment (start 128.6954 102.87) (end 133.3231 98.2423) (width 0.25) (layer "F.Cu") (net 16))
 (segment (start 133.3231 98.2423) (end 133.3231 85.0716) (width 0.25) (layer "F.Cu") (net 16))
 (segment (start 128.175 102.87) (end 128.6954 102.87) (width 0.25) (layer "F.Cu") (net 16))
 (via (at 133.3231 85.0716) (size 0.8) (drill 0.4) (layers "F.Cu" "B.Cu") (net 16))
 (segment (start 133.3231 85.0716) (end 144.78 73.6147) (width 0.25) (layer "B.Cu") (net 16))
 (segment (start 148.5049 67.31) (end 148.5049 69.85) (width 0.25) (layer "F.Cu") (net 29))
 (segment (start 148.5049 69.85) (end 145.6247 69.85) (width 0.25) (layer "F.Cu") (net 29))
 (segment (start 145.6247 69.85) (end 145.6247 70.23) (width 0.25) (layer "F.Cu") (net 29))
 (segment (start 145.6247 70.23) (end 144.78 71.0747) (width 0.25) (layer "F.Cu") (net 29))
 (segment (start 144.3885 82.55) (end 143.084 81.2455) (width 0.25) (layer "F.Cu") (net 25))
 (segment (start 148.5049 82.55) (end 144.3885 82.55) (width 0.25) (layer "F.Cu") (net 25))
 (segment (start 143.084 81.2455) (end 143.084 70.2307) (width 0.25) (layer "F.Cu") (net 25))
 (segment (start 143.084 70.2307) (end 144.78 68.5347) (width 0.25) (layer "F.Cu") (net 25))
 (segment (start 143.5241 59.6461) (end 143.5241 62.1988) (width 0.25) (layer "F.Cu") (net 32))
 (segment (start 146.0202 57.15) (end 143.5241 59.6461) (width 0.25) (layer "F.Cu") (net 32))
 (segment (start 143.5241 62.1988) (end 144.78 63.4547) (width 0.25) (layer "F.Cu") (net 32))
 (segment (start 148.1299 57.15) (end 146.0202 57.15) (width 0.25) (layer "F.Cu") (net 32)))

